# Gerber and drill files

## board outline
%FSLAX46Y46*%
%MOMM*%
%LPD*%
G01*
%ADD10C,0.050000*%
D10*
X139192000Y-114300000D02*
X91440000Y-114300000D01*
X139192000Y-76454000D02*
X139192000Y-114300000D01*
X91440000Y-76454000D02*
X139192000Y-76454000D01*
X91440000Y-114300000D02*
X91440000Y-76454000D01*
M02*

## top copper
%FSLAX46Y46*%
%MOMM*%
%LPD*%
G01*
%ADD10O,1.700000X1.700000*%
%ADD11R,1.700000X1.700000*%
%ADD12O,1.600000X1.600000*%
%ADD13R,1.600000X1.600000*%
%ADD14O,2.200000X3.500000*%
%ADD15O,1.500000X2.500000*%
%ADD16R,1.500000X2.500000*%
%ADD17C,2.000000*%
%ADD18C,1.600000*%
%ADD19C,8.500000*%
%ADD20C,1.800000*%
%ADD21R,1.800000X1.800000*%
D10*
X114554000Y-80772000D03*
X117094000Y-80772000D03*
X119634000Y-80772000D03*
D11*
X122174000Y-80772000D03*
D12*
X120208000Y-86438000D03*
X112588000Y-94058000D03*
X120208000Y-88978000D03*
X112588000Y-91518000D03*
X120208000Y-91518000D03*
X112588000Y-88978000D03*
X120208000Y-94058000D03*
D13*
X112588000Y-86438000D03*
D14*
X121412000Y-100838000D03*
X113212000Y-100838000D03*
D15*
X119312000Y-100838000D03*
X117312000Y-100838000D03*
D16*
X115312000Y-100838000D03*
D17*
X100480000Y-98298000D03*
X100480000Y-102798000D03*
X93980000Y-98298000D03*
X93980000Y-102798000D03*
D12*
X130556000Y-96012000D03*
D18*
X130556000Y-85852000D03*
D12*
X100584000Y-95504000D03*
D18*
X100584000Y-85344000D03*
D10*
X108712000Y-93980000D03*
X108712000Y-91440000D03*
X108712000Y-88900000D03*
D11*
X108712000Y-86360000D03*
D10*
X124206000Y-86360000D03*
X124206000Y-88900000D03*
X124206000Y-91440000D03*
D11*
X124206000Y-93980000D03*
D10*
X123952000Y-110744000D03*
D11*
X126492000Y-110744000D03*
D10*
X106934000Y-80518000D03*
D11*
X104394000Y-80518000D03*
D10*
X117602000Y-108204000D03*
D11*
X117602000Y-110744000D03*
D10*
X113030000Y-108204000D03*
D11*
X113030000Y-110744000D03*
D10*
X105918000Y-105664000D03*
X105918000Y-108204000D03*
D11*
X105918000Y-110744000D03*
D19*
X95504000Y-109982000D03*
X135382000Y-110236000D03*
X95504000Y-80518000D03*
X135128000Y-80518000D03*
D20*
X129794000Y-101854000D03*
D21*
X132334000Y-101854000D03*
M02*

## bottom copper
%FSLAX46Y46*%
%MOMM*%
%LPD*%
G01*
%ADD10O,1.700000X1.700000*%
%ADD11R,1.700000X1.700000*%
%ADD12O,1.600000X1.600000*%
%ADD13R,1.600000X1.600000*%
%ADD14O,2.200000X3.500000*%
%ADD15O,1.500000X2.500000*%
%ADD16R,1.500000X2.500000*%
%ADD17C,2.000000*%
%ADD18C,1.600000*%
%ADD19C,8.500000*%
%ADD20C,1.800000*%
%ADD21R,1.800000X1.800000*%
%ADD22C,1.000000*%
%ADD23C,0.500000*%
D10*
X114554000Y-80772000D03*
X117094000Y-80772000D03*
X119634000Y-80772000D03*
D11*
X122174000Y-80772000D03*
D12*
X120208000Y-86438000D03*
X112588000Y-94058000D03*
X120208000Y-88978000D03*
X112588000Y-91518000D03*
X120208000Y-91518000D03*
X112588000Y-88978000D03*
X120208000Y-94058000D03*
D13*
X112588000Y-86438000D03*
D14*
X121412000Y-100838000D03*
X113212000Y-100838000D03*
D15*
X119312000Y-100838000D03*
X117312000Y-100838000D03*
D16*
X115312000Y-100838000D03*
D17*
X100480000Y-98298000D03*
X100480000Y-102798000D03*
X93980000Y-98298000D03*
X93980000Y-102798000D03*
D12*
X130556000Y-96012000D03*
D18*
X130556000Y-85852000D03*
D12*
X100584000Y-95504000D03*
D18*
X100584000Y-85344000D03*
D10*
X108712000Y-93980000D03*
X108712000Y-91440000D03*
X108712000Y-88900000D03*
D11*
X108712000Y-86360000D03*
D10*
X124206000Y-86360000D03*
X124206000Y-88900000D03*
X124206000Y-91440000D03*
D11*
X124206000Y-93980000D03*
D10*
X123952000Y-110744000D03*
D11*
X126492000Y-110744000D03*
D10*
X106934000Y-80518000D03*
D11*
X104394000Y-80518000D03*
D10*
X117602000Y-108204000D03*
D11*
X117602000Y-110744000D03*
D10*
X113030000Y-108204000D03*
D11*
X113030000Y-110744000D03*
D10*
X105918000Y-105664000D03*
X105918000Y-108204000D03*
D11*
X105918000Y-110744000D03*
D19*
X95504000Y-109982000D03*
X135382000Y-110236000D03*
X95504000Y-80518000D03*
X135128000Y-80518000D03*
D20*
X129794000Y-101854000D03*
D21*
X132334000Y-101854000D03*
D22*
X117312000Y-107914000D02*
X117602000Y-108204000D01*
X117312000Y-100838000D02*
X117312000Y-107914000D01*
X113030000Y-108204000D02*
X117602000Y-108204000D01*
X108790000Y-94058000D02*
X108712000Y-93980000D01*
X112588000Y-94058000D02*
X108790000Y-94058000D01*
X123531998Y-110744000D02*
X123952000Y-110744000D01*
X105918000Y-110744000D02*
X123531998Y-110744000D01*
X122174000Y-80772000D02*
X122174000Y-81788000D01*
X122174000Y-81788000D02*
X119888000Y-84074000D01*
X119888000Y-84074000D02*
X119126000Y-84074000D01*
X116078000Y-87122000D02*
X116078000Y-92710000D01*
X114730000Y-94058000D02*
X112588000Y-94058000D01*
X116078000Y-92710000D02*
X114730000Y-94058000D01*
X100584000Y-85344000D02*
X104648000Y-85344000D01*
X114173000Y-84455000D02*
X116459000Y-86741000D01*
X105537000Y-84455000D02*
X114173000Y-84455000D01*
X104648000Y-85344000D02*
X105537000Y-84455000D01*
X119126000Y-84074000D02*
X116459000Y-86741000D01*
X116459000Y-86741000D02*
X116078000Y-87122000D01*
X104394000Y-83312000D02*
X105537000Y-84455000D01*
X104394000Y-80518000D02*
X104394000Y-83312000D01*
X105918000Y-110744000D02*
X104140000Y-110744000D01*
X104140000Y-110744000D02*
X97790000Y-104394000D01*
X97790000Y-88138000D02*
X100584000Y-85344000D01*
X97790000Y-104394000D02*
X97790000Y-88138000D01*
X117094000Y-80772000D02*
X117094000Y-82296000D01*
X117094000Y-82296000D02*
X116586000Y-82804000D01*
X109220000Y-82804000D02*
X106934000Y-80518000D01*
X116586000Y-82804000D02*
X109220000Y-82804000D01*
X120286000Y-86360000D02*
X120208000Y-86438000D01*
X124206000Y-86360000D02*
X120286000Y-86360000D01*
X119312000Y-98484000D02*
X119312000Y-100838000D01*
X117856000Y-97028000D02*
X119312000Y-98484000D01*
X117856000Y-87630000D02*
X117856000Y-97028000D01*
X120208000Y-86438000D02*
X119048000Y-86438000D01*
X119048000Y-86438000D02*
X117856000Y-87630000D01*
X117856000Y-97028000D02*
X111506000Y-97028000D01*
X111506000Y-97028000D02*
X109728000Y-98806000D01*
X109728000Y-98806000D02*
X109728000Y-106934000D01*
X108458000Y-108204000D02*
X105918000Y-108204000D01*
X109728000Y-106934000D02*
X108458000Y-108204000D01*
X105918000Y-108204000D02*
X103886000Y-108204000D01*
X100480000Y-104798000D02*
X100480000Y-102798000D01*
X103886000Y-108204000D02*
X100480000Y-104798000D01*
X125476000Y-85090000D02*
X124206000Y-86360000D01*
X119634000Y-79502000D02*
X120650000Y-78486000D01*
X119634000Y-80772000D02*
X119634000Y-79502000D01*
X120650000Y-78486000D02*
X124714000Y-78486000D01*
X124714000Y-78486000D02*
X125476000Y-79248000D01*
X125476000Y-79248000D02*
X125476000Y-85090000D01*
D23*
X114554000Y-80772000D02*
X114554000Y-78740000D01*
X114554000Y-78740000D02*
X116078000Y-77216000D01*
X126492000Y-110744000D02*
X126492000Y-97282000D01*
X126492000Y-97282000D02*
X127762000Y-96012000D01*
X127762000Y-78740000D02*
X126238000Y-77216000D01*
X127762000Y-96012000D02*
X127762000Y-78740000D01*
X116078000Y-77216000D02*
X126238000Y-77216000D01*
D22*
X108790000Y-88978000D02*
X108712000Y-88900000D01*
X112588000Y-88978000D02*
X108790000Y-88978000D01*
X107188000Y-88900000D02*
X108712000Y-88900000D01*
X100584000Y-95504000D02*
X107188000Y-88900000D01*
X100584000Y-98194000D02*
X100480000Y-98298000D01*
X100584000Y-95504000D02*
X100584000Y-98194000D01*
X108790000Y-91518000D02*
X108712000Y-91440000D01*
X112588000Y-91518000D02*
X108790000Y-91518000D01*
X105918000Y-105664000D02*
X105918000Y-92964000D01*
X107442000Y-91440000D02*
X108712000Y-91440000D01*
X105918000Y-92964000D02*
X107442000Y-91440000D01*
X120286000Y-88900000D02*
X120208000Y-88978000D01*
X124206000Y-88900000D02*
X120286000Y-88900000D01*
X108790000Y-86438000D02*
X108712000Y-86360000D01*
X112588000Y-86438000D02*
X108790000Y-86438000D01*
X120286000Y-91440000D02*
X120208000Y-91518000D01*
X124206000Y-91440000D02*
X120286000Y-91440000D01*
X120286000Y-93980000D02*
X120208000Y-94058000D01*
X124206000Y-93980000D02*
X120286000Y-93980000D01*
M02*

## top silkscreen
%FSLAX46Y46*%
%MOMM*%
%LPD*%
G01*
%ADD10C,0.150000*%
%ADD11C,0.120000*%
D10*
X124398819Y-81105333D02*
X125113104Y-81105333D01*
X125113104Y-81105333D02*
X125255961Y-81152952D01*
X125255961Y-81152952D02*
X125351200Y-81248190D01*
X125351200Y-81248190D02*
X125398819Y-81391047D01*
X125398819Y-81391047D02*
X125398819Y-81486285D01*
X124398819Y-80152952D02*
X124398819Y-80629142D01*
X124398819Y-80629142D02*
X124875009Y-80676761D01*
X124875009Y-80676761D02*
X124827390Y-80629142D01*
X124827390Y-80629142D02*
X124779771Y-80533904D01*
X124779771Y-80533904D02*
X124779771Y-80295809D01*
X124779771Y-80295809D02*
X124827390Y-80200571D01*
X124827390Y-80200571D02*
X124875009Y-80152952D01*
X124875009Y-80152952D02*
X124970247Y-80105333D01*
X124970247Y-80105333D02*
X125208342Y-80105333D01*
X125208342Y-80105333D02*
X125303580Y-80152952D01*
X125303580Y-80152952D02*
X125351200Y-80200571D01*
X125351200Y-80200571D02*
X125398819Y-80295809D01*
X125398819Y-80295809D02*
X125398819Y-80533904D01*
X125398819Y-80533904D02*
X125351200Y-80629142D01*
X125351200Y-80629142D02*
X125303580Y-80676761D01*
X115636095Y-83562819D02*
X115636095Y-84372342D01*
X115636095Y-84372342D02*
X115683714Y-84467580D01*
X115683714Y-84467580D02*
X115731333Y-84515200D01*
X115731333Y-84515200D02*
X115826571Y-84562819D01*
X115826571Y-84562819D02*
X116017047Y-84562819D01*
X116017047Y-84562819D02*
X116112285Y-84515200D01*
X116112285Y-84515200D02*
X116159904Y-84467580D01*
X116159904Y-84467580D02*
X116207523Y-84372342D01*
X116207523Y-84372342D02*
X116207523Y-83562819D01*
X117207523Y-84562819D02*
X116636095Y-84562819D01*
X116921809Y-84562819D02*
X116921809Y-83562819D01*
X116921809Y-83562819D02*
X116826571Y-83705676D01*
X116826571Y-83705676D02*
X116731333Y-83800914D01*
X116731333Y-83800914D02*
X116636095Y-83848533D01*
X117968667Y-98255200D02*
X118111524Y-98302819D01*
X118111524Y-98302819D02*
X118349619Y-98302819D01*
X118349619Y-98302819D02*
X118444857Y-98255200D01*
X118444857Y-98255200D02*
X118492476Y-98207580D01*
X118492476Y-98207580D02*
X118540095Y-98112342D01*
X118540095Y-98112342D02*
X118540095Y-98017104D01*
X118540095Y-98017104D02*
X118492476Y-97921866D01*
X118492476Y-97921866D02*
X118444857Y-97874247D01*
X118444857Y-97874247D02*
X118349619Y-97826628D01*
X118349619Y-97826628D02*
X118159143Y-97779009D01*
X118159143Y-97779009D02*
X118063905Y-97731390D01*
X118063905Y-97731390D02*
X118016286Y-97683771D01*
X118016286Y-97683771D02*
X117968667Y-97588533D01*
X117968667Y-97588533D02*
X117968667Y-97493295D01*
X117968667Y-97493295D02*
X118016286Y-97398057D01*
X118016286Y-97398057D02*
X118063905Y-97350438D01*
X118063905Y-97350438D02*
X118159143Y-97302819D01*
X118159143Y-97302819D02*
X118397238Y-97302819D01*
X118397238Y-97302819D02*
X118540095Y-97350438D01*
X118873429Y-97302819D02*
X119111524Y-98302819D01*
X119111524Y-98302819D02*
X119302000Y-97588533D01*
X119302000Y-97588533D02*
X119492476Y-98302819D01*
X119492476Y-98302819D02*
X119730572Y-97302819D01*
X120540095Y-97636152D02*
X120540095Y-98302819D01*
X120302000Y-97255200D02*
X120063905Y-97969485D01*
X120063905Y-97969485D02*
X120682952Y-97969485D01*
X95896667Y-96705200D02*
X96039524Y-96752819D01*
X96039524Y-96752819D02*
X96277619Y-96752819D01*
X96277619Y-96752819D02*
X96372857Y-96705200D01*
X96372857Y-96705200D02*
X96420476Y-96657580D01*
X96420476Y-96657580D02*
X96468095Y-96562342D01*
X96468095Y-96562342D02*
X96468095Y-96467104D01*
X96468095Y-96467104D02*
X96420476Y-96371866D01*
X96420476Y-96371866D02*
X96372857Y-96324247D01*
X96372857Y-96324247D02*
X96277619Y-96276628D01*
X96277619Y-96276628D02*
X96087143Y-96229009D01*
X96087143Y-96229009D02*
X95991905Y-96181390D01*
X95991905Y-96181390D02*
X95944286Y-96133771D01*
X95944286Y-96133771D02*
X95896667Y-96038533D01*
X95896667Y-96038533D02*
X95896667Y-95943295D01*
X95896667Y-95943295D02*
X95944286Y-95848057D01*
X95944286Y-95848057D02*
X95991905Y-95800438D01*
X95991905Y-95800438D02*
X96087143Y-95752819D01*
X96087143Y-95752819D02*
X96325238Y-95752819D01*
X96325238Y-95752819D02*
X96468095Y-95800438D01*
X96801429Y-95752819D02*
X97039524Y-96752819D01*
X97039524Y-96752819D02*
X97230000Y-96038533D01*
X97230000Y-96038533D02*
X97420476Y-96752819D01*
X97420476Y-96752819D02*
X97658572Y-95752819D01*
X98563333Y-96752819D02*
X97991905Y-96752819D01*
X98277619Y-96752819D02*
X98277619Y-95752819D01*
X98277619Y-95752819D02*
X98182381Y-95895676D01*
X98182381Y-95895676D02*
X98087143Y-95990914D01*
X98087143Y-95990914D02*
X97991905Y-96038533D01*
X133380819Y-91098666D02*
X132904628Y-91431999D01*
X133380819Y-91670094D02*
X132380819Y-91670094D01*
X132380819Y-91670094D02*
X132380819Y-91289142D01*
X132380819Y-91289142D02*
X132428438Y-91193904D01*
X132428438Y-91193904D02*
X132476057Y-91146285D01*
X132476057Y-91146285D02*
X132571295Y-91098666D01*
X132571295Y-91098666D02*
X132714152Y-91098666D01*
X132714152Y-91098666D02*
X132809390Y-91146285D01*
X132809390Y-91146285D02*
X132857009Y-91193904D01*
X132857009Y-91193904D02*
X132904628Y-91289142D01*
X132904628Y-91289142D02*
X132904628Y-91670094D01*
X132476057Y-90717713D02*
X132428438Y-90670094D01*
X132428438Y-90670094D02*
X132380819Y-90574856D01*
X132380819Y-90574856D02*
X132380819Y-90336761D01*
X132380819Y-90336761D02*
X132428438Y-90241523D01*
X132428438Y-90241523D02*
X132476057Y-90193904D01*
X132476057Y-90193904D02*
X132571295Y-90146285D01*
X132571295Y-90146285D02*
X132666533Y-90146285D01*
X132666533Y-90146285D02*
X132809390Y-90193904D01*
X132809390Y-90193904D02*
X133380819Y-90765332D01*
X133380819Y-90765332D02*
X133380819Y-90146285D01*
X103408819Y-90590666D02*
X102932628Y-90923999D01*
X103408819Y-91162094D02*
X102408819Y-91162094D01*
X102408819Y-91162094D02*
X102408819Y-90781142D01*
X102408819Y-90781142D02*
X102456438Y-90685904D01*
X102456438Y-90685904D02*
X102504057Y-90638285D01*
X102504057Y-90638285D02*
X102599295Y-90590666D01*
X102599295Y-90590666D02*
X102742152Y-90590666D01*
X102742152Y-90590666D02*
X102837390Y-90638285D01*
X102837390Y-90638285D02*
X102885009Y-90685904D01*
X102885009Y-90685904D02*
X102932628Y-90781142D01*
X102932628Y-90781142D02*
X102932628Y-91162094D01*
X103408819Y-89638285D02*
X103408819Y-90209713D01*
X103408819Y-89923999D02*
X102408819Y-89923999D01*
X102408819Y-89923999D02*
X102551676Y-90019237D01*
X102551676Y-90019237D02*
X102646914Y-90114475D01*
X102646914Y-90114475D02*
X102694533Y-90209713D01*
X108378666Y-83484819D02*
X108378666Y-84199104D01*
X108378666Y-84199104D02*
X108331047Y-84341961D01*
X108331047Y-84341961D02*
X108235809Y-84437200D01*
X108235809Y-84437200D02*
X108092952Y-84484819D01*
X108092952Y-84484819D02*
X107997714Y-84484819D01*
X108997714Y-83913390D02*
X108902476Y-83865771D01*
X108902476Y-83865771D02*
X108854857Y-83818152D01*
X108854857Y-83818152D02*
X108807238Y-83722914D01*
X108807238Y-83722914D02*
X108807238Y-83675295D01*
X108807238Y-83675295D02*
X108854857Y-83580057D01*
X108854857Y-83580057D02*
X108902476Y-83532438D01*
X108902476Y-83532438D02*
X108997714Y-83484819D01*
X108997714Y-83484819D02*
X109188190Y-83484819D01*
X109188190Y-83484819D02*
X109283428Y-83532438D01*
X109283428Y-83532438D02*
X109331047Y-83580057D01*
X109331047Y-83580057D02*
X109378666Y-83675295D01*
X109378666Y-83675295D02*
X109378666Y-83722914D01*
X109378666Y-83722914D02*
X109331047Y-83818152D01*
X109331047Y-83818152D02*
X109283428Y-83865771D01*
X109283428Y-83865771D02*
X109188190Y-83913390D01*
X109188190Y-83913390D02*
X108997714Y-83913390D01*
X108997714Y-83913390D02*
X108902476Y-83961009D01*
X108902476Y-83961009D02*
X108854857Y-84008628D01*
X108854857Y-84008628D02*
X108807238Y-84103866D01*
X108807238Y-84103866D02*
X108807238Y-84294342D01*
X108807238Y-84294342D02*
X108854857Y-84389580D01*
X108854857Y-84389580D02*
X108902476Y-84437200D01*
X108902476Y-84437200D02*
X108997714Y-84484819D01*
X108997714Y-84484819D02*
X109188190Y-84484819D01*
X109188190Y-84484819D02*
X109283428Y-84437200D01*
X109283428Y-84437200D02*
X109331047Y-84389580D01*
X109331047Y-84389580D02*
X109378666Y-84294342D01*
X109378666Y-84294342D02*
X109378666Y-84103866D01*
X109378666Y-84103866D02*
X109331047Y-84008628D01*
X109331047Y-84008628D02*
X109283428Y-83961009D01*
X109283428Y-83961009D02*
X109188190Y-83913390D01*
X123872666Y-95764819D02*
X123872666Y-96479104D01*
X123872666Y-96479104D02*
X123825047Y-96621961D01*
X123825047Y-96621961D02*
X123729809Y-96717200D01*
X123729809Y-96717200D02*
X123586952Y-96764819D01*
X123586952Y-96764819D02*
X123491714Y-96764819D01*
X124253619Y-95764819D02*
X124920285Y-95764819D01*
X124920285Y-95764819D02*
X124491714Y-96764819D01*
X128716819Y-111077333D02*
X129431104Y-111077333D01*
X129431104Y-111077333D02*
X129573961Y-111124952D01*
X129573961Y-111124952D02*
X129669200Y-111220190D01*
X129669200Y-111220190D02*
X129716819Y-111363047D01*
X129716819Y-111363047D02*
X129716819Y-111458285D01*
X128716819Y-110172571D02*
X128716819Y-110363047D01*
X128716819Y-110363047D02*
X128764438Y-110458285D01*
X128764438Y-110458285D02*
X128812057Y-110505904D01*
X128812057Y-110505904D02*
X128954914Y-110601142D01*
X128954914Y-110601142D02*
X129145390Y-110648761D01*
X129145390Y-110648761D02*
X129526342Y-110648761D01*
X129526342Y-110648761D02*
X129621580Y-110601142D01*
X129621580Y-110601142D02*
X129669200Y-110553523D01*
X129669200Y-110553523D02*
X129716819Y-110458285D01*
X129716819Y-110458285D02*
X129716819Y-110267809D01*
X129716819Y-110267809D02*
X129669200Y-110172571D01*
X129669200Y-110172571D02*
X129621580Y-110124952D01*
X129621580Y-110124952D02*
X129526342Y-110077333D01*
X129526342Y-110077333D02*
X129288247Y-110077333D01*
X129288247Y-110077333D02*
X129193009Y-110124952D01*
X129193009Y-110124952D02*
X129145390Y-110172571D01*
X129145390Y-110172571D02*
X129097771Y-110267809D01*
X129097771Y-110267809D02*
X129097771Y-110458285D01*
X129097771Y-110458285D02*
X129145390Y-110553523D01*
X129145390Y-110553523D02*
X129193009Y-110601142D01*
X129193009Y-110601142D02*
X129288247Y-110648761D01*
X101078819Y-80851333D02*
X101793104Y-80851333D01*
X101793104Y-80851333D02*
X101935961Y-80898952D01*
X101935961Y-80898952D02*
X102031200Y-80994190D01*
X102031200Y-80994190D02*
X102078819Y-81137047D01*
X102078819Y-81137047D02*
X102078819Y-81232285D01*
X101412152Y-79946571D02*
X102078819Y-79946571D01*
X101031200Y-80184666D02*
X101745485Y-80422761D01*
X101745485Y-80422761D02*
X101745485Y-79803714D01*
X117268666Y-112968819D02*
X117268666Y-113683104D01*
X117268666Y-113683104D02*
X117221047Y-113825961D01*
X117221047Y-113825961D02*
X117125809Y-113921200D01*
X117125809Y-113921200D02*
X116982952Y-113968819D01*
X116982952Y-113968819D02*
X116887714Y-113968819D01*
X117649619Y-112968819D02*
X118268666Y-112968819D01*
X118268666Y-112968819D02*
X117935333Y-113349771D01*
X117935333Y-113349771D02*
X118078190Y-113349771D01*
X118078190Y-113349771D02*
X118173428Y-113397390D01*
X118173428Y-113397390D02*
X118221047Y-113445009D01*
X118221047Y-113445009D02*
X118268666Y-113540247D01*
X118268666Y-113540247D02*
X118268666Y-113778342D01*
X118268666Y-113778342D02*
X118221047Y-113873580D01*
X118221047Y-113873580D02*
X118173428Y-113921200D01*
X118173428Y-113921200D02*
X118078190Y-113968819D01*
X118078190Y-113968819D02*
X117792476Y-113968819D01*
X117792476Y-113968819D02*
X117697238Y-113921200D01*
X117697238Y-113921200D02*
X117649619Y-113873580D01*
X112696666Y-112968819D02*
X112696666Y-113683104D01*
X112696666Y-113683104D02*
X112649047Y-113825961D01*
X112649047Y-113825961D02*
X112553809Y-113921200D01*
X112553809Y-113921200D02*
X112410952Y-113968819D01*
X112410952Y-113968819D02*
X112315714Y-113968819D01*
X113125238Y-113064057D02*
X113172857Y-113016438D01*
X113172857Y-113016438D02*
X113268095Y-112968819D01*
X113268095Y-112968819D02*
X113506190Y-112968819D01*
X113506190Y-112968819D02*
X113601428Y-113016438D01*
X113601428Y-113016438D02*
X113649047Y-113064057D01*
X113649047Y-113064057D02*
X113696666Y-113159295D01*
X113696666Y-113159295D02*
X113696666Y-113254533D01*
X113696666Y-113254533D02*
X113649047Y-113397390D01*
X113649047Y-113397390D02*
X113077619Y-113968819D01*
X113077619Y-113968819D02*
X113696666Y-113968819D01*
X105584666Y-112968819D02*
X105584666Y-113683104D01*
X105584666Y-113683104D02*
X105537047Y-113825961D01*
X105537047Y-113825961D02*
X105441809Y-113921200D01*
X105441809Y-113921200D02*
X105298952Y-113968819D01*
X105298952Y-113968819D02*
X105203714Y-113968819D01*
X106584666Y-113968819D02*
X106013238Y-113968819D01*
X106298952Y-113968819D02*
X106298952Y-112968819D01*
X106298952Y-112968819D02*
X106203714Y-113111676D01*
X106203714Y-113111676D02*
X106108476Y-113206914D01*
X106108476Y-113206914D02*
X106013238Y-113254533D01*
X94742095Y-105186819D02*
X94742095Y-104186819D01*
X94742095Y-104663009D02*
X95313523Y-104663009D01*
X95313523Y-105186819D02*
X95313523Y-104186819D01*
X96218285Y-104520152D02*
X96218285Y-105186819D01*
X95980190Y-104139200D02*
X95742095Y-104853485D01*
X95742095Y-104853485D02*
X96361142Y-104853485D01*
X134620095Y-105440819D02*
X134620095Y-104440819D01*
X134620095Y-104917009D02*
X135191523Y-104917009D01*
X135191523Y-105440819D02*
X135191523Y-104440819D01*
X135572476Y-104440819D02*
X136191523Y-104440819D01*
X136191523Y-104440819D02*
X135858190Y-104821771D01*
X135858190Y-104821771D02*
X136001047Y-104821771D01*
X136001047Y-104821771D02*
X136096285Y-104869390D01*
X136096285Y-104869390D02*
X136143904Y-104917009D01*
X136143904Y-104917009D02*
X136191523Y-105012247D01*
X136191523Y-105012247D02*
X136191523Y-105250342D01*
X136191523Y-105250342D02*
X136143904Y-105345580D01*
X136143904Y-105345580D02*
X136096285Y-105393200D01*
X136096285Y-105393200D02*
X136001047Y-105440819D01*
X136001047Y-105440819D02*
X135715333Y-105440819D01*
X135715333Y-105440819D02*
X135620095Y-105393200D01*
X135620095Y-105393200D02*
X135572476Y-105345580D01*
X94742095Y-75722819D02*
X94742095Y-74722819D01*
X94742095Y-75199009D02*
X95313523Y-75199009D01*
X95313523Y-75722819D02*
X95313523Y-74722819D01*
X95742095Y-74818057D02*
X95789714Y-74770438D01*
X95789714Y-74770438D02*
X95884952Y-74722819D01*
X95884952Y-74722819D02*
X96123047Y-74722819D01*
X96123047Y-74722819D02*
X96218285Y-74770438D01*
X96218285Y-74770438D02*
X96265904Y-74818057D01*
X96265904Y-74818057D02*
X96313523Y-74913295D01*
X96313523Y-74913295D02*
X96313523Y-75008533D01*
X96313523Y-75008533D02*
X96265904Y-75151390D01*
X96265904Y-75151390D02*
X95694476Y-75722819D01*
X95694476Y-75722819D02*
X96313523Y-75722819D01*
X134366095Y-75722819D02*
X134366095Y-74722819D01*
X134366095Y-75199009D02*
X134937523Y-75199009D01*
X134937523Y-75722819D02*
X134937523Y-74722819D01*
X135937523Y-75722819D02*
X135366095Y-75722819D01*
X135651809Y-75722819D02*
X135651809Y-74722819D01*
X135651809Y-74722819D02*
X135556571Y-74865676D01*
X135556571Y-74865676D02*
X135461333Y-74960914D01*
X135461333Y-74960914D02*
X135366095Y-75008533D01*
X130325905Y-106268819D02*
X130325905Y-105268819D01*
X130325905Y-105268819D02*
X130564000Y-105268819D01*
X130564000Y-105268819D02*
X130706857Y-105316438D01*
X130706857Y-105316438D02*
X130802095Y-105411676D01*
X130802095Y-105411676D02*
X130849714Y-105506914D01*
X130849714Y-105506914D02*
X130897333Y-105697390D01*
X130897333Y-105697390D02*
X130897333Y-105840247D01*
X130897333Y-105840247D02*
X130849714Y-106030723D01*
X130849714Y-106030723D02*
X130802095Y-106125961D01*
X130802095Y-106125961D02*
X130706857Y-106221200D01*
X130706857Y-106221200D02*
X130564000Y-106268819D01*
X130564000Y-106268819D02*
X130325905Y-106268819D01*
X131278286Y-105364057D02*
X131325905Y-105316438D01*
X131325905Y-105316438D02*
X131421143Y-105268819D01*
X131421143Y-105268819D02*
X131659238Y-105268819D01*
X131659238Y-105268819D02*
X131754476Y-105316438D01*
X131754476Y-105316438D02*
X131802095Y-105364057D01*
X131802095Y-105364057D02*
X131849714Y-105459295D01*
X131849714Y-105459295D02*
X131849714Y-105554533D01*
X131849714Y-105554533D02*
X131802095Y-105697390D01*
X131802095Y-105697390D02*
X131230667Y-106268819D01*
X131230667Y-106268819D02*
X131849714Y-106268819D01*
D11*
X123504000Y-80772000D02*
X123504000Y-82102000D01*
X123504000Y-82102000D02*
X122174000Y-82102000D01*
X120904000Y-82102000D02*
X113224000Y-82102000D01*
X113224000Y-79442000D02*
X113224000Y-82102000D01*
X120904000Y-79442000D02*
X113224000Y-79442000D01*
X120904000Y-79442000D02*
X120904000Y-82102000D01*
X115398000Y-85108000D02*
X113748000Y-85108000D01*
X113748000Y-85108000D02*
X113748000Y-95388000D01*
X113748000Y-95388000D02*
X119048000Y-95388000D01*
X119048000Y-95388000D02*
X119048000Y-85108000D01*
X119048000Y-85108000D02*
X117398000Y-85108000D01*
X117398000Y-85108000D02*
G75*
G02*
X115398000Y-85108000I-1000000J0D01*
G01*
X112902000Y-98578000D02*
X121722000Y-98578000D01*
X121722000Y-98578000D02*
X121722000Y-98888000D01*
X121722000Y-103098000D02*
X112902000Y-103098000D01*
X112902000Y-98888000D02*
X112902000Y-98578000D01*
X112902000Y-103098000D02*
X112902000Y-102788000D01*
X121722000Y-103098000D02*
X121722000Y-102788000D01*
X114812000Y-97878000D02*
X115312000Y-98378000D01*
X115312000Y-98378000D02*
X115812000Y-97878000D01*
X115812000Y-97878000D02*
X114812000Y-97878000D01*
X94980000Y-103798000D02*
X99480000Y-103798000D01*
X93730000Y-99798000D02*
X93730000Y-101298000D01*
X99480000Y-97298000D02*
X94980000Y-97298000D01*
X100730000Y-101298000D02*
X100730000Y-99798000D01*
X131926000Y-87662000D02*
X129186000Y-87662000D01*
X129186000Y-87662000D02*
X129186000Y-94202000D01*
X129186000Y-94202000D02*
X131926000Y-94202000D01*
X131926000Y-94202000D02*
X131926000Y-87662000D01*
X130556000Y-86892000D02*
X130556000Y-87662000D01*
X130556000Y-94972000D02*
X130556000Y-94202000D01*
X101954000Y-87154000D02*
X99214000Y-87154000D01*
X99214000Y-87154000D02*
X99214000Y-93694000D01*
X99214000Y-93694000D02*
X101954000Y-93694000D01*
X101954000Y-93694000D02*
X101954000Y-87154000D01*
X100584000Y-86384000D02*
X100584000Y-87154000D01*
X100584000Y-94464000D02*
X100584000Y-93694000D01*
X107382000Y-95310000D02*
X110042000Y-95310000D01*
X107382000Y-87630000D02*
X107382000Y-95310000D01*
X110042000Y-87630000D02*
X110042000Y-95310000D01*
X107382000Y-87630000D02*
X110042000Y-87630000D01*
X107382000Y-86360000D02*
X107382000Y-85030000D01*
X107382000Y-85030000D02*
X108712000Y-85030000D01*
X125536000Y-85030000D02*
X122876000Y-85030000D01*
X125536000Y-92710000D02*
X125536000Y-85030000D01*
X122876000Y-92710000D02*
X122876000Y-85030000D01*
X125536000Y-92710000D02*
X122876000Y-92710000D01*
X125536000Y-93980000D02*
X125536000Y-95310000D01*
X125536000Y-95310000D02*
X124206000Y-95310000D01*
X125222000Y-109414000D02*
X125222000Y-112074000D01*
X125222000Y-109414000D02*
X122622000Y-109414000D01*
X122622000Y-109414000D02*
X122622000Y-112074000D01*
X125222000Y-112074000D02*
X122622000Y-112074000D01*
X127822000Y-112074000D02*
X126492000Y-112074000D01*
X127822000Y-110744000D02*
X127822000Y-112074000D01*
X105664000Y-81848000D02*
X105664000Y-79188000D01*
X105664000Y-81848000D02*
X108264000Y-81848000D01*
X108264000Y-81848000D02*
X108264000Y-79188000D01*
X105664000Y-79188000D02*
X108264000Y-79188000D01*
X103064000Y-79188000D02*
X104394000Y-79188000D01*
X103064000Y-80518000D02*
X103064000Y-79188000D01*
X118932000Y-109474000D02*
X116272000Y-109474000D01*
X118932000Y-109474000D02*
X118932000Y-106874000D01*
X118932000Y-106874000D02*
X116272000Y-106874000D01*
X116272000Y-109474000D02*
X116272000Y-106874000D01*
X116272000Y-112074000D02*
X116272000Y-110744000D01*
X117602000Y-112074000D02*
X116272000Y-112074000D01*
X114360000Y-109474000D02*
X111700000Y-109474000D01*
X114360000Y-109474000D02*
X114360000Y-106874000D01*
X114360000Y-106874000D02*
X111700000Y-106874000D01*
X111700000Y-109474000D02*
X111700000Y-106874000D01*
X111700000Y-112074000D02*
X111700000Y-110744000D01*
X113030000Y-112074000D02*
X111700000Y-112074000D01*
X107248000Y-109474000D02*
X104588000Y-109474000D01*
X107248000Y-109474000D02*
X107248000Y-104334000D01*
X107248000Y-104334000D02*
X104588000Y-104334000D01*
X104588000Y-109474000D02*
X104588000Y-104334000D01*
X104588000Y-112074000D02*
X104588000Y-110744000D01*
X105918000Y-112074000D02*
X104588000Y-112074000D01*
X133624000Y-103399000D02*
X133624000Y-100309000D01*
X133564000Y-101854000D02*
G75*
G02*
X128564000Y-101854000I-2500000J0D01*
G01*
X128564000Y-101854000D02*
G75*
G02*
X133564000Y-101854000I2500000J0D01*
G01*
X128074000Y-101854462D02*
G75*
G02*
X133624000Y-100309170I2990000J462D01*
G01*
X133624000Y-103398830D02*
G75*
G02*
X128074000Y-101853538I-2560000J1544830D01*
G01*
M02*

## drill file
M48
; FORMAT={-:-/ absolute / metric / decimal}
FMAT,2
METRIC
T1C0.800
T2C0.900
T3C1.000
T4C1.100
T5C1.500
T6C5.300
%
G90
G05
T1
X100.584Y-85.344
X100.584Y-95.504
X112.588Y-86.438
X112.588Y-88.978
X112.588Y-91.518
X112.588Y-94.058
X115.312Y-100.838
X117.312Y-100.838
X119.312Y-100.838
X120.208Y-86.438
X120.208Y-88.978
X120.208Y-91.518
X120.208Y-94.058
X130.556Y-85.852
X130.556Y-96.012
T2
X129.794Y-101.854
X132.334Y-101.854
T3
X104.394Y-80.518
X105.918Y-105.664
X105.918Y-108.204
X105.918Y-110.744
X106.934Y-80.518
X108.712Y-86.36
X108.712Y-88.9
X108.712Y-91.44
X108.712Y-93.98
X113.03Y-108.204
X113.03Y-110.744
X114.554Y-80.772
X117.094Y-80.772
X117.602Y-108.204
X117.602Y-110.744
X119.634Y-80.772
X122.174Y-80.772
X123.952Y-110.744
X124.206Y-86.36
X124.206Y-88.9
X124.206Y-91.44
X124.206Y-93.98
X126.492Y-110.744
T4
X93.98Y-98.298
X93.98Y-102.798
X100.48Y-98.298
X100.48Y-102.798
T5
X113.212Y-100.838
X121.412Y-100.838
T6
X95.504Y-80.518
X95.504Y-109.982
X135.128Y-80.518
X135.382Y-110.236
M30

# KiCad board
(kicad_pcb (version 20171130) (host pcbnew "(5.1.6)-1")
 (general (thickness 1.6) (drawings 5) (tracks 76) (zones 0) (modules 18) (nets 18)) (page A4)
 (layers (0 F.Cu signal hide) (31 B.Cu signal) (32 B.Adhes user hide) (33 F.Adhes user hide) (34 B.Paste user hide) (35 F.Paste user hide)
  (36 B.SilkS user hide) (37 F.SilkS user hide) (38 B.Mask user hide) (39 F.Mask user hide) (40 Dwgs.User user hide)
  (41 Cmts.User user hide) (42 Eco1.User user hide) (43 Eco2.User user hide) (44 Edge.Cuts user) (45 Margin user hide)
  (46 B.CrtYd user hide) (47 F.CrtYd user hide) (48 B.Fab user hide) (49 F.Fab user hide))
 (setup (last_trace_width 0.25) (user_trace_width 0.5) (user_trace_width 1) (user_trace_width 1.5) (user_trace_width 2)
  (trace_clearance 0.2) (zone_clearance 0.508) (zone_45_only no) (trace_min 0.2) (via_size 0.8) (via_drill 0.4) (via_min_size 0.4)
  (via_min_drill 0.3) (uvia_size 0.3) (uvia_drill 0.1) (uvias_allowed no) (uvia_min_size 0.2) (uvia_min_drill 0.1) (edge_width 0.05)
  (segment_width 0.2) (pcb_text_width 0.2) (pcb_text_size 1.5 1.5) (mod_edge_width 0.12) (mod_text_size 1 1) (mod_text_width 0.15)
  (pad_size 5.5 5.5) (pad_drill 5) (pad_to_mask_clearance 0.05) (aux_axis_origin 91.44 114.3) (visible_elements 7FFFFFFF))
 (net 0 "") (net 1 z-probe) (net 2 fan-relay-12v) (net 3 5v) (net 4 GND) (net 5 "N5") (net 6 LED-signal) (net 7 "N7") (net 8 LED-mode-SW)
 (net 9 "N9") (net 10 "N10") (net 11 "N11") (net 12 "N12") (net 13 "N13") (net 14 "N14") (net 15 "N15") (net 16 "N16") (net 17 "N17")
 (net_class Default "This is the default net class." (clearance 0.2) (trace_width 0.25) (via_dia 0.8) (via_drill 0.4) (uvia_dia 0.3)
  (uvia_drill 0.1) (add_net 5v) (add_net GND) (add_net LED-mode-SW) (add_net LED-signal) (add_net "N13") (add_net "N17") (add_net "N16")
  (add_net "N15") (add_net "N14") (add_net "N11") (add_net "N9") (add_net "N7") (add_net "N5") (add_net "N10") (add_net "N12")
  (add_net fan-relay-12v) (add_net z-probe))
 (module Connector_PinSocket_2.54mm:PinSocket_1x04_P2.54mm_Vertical (layer F.Cu) (at 122.174 80.772 270)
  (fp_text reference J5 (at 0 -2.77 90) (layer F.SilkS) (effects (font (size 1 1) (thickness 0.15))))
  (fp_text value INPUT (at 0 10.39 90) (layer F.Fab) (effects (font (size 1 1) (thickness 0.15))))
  (fp_line (start 0 -1.33) (end 1.33 -1.33) (layer F.SilkS) (width 0.12))
  (fp_line (start 1.33 -1.33) (end 1.33 0) (layer F.SilkS) (width 0.12))
  (fp_line (start 1.33 1.27) (end 1.33 8.95) (layer F.SilkS) (width 0.12))
  (fp_line (start -1.33 8.95) (end 1.33 8.95) (layer F.SilkS) (width 0.12))
  (fp_line (start -1.33 1.27) (end -1.33 8.95) (layer F.SilkS) (width 0.12))
  (fp_line (start -1.33 1.27) (end 1.33 1.27) (layer F.SilkS) (width 0.12))
  (pad 4 thru_hole oval (at 0 7.62 270) (size 1.7 1.7) (drill 1) (layers *.Cu *.Mask) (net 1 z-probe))
  (pad 3 thru_hole oval (at 0 5.08 270) (size 1.7 1.7) (drill 1) (layers *.Cu *.Mask) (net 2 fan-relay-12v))
  (pad 2 thru_hole oval (at 0 2.54 270) (size 1.7 1.7) (drill 1) (layers *.Cu *.Mask) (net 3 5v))
  (pad 1 thru_hole rect (at 0 0 270) (size 1.7 1.7) (drill 1) (layers *.Cu *.Mask) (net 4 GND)))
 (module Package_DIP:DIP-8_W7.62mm (layer F.Cu) (at 112.588 86.438)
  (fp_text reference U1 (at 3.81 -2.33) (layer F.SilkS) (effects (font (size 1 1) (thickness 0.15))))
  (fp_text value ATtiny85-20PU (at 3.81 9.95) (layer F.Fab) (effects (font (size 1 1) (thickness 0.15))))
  (fp_line (start 2.81 -1.33) (end 1.16 -1.33) (layer F.SilkS) (width 0.12))
  (fp_line (start 1.16 -1.33) (end 1.16 8.95) (layer F.SilkS) (width 0.12))
  (fp_line (start 1.16 8.95) (end 6.46 8.95) (layer F.SilkS) (width 0.12))
  (fp_line (start 6.46 8.95) (end 6.46 -1.33) (layer F.SilkS) (width 0.12))
  (fp_line (start 6.46 -1.33) (end 4.81 -1.33) (layer F.SilkS) (width 0.12))
  (fp_arc (start 3.81 -1.33) (end 2.81 -1.33) (angle -180) (layer F.SilkS) (width 0.12))
  (pad 8 thru_hole oval (at 7.62 0) (size 1.6 1.6) (drill 0.8) (layers *.Cu *.Mask) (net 3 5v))
  (pad 4 thru_hole oval (at 0 7.62) (size 1.6 1.6) (drill 0.8) (layers *.Cu *.Mask) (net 4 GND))
  (pad 7 thru_hole oval (at 7.62 2.54) (size 1.6 1.6) (drill 0.8) (layers *.Cu *.Mask) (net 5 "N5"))
  (pad 3 thru_hole oval (at 0 5.08) (size 1.6 1.6) (drill 0.8) (layers *.Cu *.Mask) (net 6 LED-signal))
  (pad 6 thru_hole oval (at 7.62 5.08) (size 1.6 1.6) (drill 0.8) (layers *.Cu *.Mask) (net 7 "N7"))
  (pad 2 thru_hole oval (at 0 2.54) (size 1.6 1.6) (drill 0.8) (layers *.Cu *.Mask) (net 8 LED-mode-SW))
  (pad 5 thru_hole oval (at 7.62 7.62) (size 1.6 1.6) (drill 0.8) (layers *.Cu *.Mask) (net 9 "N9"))
  (pad 1 thru_hole rect (at 0 0) (size 1.6 1.6) (drill 0.8) (layers *.Cu *.Mask) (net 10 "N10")))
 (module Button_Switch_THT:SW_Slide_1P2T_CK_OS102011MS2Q (layer F.Cu) (at 115.312 100.838)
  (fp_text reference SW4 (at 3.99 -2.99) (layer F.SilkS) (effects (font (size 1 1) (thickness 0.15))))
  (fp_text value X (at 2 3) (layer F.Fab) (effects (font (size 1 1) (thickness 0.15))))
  (fp_line (start -2.41 -2.26) (end 6.41 -2.26) (layer F.SilkS) (width 0.12))
  (fp_line (start 6.41 -2.26) (end 6.41 -1.95) (layer F.SilkS) (width 0.12))
  (fp_line (start 6.41 2.26) (end -2.41 2.26) (layer F.SilkS) (width 0.12))
  (fp_line (start -2.41 -1.95) (end -2.41 -2.26) (layer F.SilkS) (width 0.12))
  (fp_line (start -2.41 2.26) (end -2.41 1.95) (layer F.SilkS) (width 0.12))
  (fp_line (start 6.41 2.26) (end 6.41 1.95) (layer F.SilkS) (width 0.12))
  (fp_line (start -0.5 -2.96) (end 0 -2.46) (layer F.SilkS) (width 0.12))
  (fp_line (start 0 -2.46) (end 0.5 -2.96) (layer F.SilkS) (width 0.12))
  (fp_line (start 0.5 -2.96) (end -0.5 -2.96) (layer F.SilkS) (width 0.12))
  (pad "" thru_hole oval (at 6.1 0) (size 2.2 3.5) (drill 1.5) (layers *.Cu *.Mask))
  (pad "" thru_hole oval (at -2.1 0) (size 2.2 3.5) (drill 1.5) (layers *.Cu *.Mask))
  (pad 3 thru_hole oval (at 4 0) (size 1.5 2.5) (drill 0.8) (layers *.Cu *.Mask) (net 3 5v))
  (pad 2 thru_hole oval (at 2 0) (size 1.5 2.5) (drill 0.8) (layers *.Cu *.Mask) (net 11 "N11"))
  (pad 1 thru_hole rect (at 0 0) (size 1.5 2.5) (drill 0.8) (layers *.Cu *.Mask) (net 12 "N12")))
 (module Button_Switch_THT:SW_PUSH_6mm (layer F.Cu) (at 93.98 98.298)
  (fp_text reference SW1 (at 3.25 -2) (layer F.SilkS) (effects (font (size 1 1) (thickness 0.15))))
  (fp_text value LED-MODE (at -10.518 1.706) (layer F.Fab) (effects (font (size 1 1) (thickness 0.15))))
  (fp_line (start 1 5.5) (end 5.5 5.5) (layer F.SilkS) (width 0.12))
  (fp_line (start -0.25 1.5) (end -0.25 3) (layer F.SilkS) (width 0.12))
  (fp_line (start 5.5 -1) (end 1 -1) (layer F.SilkS) (width 0.12))
  (fp_line (start 6.75 3) (end 6.75 1.5) (layer F.SilkS) (width 0.12))
  (pad 1 thru_hole circle (at 6.5 0 90) (size 2 2) (drill 1.1) (layers *.Cu *.Mask) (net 8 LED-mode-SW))
  (pad 2 thru_hole circle (at 6.5 4.5 90) (size 2 2) (drill 1.1) (layers *.Cu *.Mask) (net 3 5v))
  (pad 1 thru_hole circle (at 0 0 90) (size 2 2) (drill 1.1) (layers *.Cu *.Mask) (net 8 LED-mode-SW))
  (pad 2 thru_hole circle (at 0 4.5 90) (size 2 2) (drill 1.1) (layers *.Cu *.Mask) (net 3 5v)))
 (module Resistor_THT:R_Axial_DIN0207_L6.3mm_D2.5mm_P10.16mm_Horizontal (layer F.Cu) (at 130.556 85.852 270)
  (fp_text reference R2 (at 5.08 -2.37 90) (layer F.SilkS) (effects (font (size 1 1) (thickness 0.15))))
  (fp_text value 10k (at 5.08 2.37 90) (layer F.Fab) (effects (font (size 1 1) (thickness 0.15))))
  (fp_line (start 1.81 -1.37) (end 1.81 1.37) (layer F.SilkS) (width 0.12))
  (fp_line (start 1.81 1.37) (end 8.35 1.37) (layer F.SilkS) (width 0.12))
  (fp_line (start 8.35 1.37) (end 8.35 -1.37) (layer F.SilkS) (width 0.12))
  (fp_line (start 8.35 -1.37) (end 1.81 -1.37) (layer F.SilkS) (width 0.12))
  (fp_line (start 1.04 0) (end 1.81 0) (layer F.SilkS) (width 0.12))
  (fp_line (start 9.12 0) (end 8.35 0) (layer F.SilkS) (width 0.12))
  (pad 2 thru_hole oval (at 10.16 0 270) (size 1.6 1.6) (drill 0.8) (layers *.Cu *.Mask) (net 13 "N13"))
  (pad 1 thru_hole circle (at 0 0 270) (size 1.6 1.6) (drill 0.8) (layers *.Cu *.Mask) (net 3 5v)))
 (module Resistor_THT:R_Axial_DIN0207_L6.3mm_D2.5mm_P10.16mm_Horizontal (layer F.Cu) (at 100.584 85.344 270)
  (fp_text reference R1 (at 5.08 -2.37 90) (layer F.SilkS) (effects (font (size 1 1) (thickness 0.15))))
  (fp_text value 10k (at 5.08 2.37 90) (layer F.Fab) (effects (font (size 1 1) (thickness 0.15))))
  (fp_line (start 1.81 -1.37) (end 1.81 1.37) (layer F.SilkS) (width 0.12))
  (fp_line (start 1.81 1.37) (end 8.35 1.37) (layer F.SilkS) (width 0.12))
  (fp_line (start 8.35 1.37) (end 8.35 -1.37) (layer F.SilkS) (width 0.12))
  (fp_line (start 8.35 -1.37) (end 1.81 -1.37) (layer F.SilkS) (width 0.12))
  (fp_line (start 1.04 0) (end 1.81 0) (layer F.SilkS) (width 0.12))
  (fp_line (start 9.12 0) (end 8.35 0) (layer F.SilkS) (width 0.12))
  (pad 2 thru_hole oval (at 10.16 0 270) (size 1.6 1.6) (drill 0.8) (layers *.Cu *.Mask) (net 8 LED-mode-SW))
  (pad 1 thru_hole circle (at 0 0 270) (size 1.6 1.6) (drill 0.8) (layers *.Cu *.Mask) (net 4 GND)))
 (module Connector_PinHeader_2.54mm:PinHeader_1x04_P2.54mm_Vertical (layer F.Cu) (at 108.712 86.36)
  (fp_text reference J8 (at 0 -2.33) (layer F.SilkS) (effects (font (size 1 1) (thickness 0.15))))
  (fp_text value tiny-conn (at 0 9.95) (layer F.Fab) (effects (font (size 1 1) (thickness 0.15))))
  (fp_line (start -1.33 8.95) (end 1.33 8.95) (layer F.SilkS) (width 0.12))
  (fp_line (start -1.33 1.27) (end -1.33 8.95) (layer F.SilkS) (width 0.12))
  (fp_line (start 1.33 1.27) (end 1.33 8.95) (layer F.SilkS) (width 0.12))
  (fp_line (start -1.33 1.27) (end 1.33 1.27) (layer F.SilkS) (width 0.12))
  (fp_line (start -1.33 0) (end -1.33 -1.33) (layer F.SilkS) (width 0.12))
  (fp_line (start -1.33 -1.33) (end 0 -1.33) (layer F.SilkS) (width 0.12))
  (pad 4 thru_hole oval (at 0 7.62) (size 1.7 1.7) (drill 1) (layers *.Cu *.Mask) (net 4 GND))
  (pad 3 thru_hole oval (at 0 5.08) (size 1.7 1.7) (drill 1) (layers *.Cu *.Mask) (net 6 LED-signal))
  (pad 2 thru_hole oval (at 0 2.54) (size 1.7 1.7) (drill 1) (layers *.Cu *.Mask) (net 8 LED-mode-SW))
  (pad 1 thru_hole rect (at 0 0) (size 1.7 1.7) (drill 1) (layers *.Cu *.Mask) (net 10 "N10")))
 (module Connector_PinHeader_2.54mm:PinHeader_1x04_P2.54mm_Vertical (layer F.Cu) (at 124.206 93.98 180)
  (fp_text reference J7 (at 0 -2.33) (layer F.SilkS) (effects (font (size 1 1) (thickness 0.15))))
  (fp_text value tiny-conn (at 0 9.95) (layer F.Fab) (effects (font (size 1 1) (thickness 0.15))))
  (fp_line (start -1.33 8.95) (end 1.33 8.95) (layer F.SilkS) (width 0.12))
  (fp_line (start -1.33 1.27) (end -1.33 8.95) (layer F.SilkS) (width 0.12))
  (fp_line (start 1.33 1.27) (end 1.33 8.95) (layer F.SilkS) (width 0.12))
  (fp_line (start -1.33 1.27) (end 1.33 1.27) (layer F.SilkS) (width 0.12))
  (fp_line (start -1.33 0) (end -1.33 -1.33) (layer F.SilkS) (width 0.12))
  (fp_line (start -1.33 -1.33) (end 0 -1.33) (layer F.SilkS) (width 0.12))
  (pad 4 thru_hole oval (at 0 7.62 180) (size 1.7 1.7) (drill 1) (layers *.Cu *.Mask) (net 3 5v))
  (pad 3 thru_hole oval (at 0 5.08 180) (size 1.7 1.7) (drill 1) (layers *.Cu *.Mask) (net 5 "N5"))
  (pad 2 thru_hole oval (at 0 2.54 180) (size 1.7 1.7) (drill 1) (layers *.Cu *.Mask) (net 7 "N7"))
  (pad 1 thru_hole rect (at 0 0 180) (size 1.7 1.7) (drill 1) (layers *.Cu *.Mask) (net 9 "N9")))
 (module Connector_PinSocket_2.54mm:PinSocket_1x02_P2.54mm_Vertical (layer F.Cu) (at 126.492 110.744 270)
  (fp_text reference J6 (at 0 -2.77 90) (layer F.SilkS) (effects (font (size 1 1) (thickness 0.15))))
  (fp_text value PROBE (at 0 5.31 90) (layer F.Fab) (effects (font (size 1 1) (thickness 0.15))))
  (fp_line (start -1.33 1.27) (end 1.33 1.27) (layer F.SilkS) (width 0.12))
  (fp_line (start -1.33 1.27) (end -1.33 3.87) (layer F.SilkS) (width 0.12))
  (fp_line (start -1.33 3.87) (end 1.33 3.87) (layer F.SilkS) (width 0.12))
  (fp_line (start 1.33 1.27) (end 1.33 3.87) (layer F.SilkS) (width 0.12))
  (fp_line (start 1.33 -1.33) (end 1.33 0) (layer F.SilkS) (width 0.12))
  (fp_line (start 0 -1.33) (end 1.33 -1.33) (layer F.SilkS) (width 0.12))
  (pad 2 thru_hole oval (at 0 2.54 270) (size 1.7 1.7) (drill 1) (layers *.Cu *.Mask) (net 4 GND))
  (pad 1 thru_hole rect (at 0 0 270) (size 1.7 1.7) (drill 1) (layers *.Cu *.Mask) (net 1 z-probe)))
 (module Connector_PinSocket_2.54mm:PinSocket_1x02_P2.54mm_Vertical (layer F.Cu) (at 104.394 80.518 90)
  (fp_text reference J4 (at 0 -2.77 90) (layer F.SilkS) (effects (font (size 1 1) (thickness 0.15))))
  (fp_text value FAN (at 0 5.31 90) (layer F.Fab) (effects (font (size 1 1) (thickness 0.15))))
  (fp_line (start -1.33 1.27) (end 1.33 1.27) (layer F.SilkS) (width 0.12))
  (fp_line (start -1.33 1.27) (end -1.33 3.87) (layer F.SilkS) (width 0.12))
  (fp_line (start -1.33 3.87) (end 1.33 3.87) (layer F.SilkS) (width 0.12))
  (fp_line (start 1.33 1.27) (end 1.33 3.87) (layer F.SilkS) (width 0.12))
  (fp_line (start 1.33 -1.33) (end 1.33 0) (layer F.SilkS) (width 0.12))
  (fp_line (start 0 -1.33) (end 1.33 -1.33) (layer F.SilkS) (width 0.12))
  (pad 2 thru_hole oval (at 0 2.54 90) (size 1.7 1.7) (drill 1) (layers *.Cu *.Mask) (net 2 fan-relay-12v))
  (pad 1 thru_hole rect (at 0 0 90) (size 1.7 1.7) (drill 1) (layers *.Cu *.Mask) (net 4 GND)))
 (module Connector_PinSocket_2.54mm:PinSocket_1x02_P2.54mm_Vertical (layer F.Cu) (at 117.602 110.744 180)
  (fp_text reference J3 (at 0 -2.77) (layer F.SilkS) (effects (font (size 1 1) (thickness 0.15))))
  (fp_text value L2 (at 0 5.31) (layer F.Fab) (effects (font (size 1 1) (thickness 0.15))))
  (fp_line (start -1.33 1.27) (end 1.33 1.27) (layer F.SilkS) (width 0.12))
  (fp_line (start -1.33 1.27) (end -1.33 3.87) (layer F.SilkS) (width 0.12))
  (fp_line (start -1.33 3.87) (end 1.33 3.87) (layer F.SilkS) (width 0.12))
  (fp_line (start 1.33 1.27) (end 1.33 3.87) (layer F.SilkS) (width 0.12))
  (fp_line (start 1.33 -1.33) (end 1.33 0) (layer F.SilkS) (width 0.12))
  (fp_line (start 0 -1.33) (end 1.33 -1.33) (layer F.SilkS) (width 0.12))
  (pad 2 thru_hole oval (at 0 2.54 180) (size 1.7 1.7) (drill 1) (layers *.Cu *.Mask) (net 11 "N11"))
  (pad 1 thru_hole rect (at 0 0 180) (size 1.7 1.7) (drill 1) (layers *.Cu *.Mask) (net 4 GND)))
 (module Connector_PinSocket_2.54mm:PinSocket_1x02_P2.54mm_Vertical (layer F.Cu) (at 113.03 110.744 180)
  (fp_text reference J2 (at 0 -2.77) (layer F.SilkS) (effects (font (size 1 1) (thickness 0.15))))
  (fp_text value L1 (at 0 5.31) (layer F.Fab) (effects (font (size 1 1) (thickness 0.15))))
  (fp_line (start -1.33 1.27) (end 1.33 1.27) (layer F.SilkS) (width 0.12))
  (fp_line (start -1.33 1.27) (end -1.33 3.87) (layer F.SilkS) (width 0.12))
  (fp_line (start -1.33 3.87) (end 1.33 3.87) (layer F.SilkS) (width 0.12))
  (fp_line (start 1.33 1.27) (end 1.33 3.87) (layer F.SilkS) (width 0.12))
  (fp_line (start 1.33 -1.33) (end 1.33 0) (layer F.SilkS) (width 0.12))
  (fp_line (start 0 -1.33) (end 1.33 -1.33) (layer F.SilkS) (width 0.12))
  (pad 2 thru_hole oval (at 0 2.54 180) (size 1.7 1.7) (drill 1) (layers *.Cu *.Mask) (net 11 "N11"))
  (pad 1 thru_hole rect (at 0 0 180) (size 1.7 1.7) (drill 1) (layers *.Cu *.Mask) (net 4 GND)))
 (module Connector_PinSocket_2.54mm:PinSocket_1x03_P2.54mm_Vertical (layer F.Cu) (at 105.918 110.744 180)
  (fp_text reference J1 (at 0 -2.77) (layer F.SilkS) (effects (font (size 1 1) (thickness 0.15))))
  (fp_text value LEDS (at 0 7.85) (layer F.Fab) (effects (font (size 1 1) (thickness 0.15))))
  (fp_line (start -1.33 1.27) (end 1.33 1.27) (layer F.SilkS) (width 0.12))
  (fp_line (start -1.33 1.27) (end -1.33 6.41) (layer F.SilkS) (width 0.12))
  (fp_line (start -1.33 6.41) (end 1.33 6.41) (layer F.SilkS) (width 0.12))
  (fp_line (start 1.33 1.27) (end 1.33 6.41) (layer F.SilkS) (width 0.12))
  (fp_line (start 1.33 -1.33) (end 1.33 0) (layer F.SilkS) (width 0.12))
  (fp_line (start 0 -1.33) (end 1.33 -1.33) (layer F.SilkS) (width 0.12))
  (pad 3 thru_hole oval (at 0 5.08 180) (size 1.7 1.7) (drill 1) (layers *.Cu *.Mask) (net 6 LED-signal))
  (pad 2 thru_hole oval (at 0 2.54 180) (size 1.7 1.7) (drill 1) (layers *.Cu *.Mask) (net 3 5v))
  (pad 1 thru_hole rect (at 0 0 180) (size 1.7 1.7) (drill 1) (layers *.Cu *.Mask) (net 4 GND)))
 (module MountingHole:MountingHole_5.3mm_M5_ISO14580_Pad (layer F.Cu) (at 95.504 109.982)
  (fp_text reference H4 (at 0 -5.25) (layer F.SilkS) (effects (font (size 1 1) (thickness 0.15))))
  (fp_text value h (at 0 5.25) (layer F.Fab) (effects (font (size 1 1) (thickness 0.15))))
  (pad 1 thru_hole circle (at 0 0) (size 8.5 8.5) (drill 5.3) (layers *.Cu *.Mask) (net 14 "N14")))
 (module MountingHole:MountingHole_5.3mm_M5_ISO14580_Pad (layer F.Cu) (at 135.382 110.236)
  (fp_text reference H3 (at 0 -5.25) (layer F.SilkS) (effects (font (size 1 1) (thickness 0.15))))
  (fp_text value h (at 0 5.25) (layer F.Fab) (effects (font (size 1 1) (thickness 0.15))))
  (pad 1 thru_hole circle (at 0 0) (size 8.5 8.5) (drill 5.3) (layers *.Cu *.Mask) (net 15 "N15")))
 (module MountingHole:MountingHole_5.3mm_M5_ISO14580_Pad (layer F.Cu) (at 95.504 80.518)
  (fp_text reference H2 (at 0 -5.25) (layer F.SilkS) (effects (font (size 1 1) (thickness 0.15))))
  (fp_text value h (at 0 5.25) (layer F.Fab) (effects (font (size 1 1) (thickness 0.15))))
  (pad 1 thru_hole circle (at 0 0) (size 8.5 8.5) (drill 5.3) (layers *.Cu *.Mask) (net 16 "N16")))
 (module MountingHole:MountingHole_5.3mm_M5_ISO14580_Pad (layer F.Cu) (at 135.128 80.518)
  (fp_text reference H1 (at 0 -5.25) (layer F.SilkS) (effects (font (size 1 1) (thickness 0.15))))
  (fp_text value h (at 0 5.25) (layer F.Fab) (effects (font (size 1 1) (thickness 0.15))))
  (pad 1 thru_hole circle (at 0 0) (size 8.5 8.5) (drill 5.3) (layers *.Cu *.Mask) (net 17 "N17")))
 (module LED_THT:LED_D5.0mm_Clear (layer F.Cu) (at 132.334 101.854 180)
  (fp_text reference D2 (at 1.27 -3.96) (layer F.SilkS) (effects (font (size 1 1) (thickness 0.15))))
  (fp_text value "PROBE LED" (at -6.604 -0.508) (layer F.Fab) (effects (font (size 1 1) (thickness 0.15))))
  (fp_line (start -1.29 -1.545) (end -1.29 1.545) (layer F.SilkS) (width 0.12))
  (fp_circle (center 1.27 0) (end 3.77 0) (layer F.SilkS) (width 0.12))
  (fp_arc (start 1.27 0) (end -1.29 1.54483) (angle -148.9) (layer F.SilkS) (width 0.12))
  (fp_arc (start 1.27 0) (end -1.29 -1.54483) (angle 148.9) (layer F.SilkS) (width 0.12))
  (pad 2 thru_hole circle (at 2.54 0 180) (size 1.8 1.8) (drill 0.9) (layers *.Cu *.Mask) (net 1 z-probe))
  (pad 1 thru_hole rect (at 0 0 180) (size 1.8 1.8) (drill 0.9) (layers *.Cu *.Mask) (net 13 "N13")))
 (gr_line (start 139.192 114.3) (end 91.44 114.3) (layer Edge.Cuts) (width 0.05))
 (gr_line (start 139.192 76.454) (end 139.192 114.3) (layer Edge.Cuts) (width 0.05))
 (gr_line (start 91.44 76.454) (end 139.192 76.454) (layer Edge.Cuts) (width 0.05))
 (gr_line (start 91.44 114.3) (end 91.44 76.454) (layer Edge.Cuts) (width 0.05))
 (segment (start 117.312 107.914) (end 117.602 108.204) (width 1) (layer B.Cu) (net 11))
 (segment (start 117.312 100.838) (end 117.312 107.914) (width 1) (layer B.Cu) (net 11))
 (segment (start 113.03 108.204) (end 117.602 108.204) (width 1) (layer B.Cu) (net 11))
 (segment (start 108.79 94.058) (end 108.712 93.98) (width 1) (layer B.Cu) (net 4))
 (segment (start 112.588 94.058) (end 108.79 94.058) (width 1) (layer B.Cu) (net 4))
 (segment (start 123.531998 110.744) (end 123.952 110.744) (width 1) (layer B.Cu) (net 4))
 (segment (start 105.918 110.744) (end 123.531998 110.744) (width 1) (layer B.Cu) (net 4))
 (segment (start 122.174 80.772) (end 122.174 81.788) (width 1) (layer B.Cu) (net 4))
 (segment (start 122.174 81.788) (end 119.888 84.074) (width 1) (layer B.Cu) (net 4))
 (segment (start 119.888 84.074) (end 119.126 84.074) (width 1) (layer B.Cu) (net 4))
 (segment (start 116.078 87.122) (end 116.078 92.71) (width 1) (layer B.Cu) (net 4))
 (segment (start 114.73 94.058) (end 112.588 94.058) (width 1) (layer B.Cu) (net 4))
 (segment (start 116.078 92.71) (end 114.73 94.058) (width 1) (layer B.Cu) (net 4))
 (segment (start 100.584 85.344) (end 104.648 85.344) (width 1) (layer B.Cu) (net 4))
 (segment (start 114.173 84.455) (end 116.459 86.741) (width 1) (layer B.Cu) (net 4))
 (segment (start 105.537 84.455) (end 114.173 84.455) (width 1) (layer B.Cu) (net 4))
 (segment (start 104.648 85.344) (end 105.537 84.455) (width 1) (layer B.Cu) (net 4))
 (segment (start 119.126 84.074) (end 116.459 86.741) (width 1) (layer B.Cu) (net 4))
 (segment (start 116.459 86.741) (end 116.078 87.122) (width 1) (layer B.Cu) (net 4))
 (segment (start 104.394 83.312) (end 105.537 84.455) (width 1) (layer B.Cu) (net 4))
 (segment (start 104.394 80.518) (end 104.394 83.312) (width 1) (layer B.Cu) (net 4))
 (segment (start 105.918 110.744) (end 104.14 110.744) (width 1) (layer B.Cu) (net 4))
 (segment (start 104.14 110.744) (end 97.79 104.394) (width 1) (layer B.Cu) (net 4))
 (segment (start 97.79 88.138) (end 100.584 85.344) (width 1) (layer B.Cu) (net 4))
 (segment (start 97.79 104.394) (end 97.79 88.138) (width 1) (layer B.Cu) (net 4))
 (segment (start 117.094 80.772) (end 117.094 82.296) (width 1) (layer B.Cu) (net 2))
 (segment (start 117.094 82.296) (end 116.586 82.804) (width 1) (layer B.Cu) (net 2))
 (segment (start 109.22 82.804) (end 106.934 80.518) (width 1) (layer B.Cu) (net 2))
 (segment (start 116.586 82.804) (end 109.22 82.804) (width 1) (layer B.Cu) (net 2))
 (segment (start 120.286 86.36) (end 120.208 86.438) (width 1) (layer B.Cu) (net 3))
 (segment (start 124.206 86.36) (end 120.286 86.36) (width 1) (layer B.Cu) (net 3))
 (segment (start 119.312 98.484) (end 119.312 100.838) (width 1) (layer B.Cu) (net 3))
 (segment (start 117.856 97.028) (end 119.312 98.484) (width 1) (layer B.Cu) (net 3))
 (segment (start 117.856 87.63) (end 117.856 97.028) (width 1) (layer B.Cu) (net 3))
 (segment (start 120.208 86.438) (end 119.048 86.438) (width 1) (layer B.Cu) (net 3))
 (segment (start 119.048 86.438) (end 117.856 87.63) (width 1) (layer B.Cu) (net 3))
 (segment (start 117.856 97.028) (end 111.506 97.028) (width 1) (layer B.Cu) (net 3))
 (segment (start 111.506 97.028) (end 109.728 98.806) (width 1) (layer B.Cu) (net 3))
 (segment (start 109.728 98.806) (end 109.728 106.934) (width 1) (layer B.Cu) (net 3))
 (segment (start 108.458 108.204) (end 105.918 108.204) (width 1) (layer B.Cu) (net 3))
 (segment (start 109.728 106.934) (end 108.458 108.204) (width 1) (layer B.Cu) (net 3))
 (segment (start 105.918 108.204) (end 103.886 108.204) (width 1) (layer B.Cu) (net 3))
 (segment (start 100.48 104.798) (end 100.48 102.798) (width 1) (layer B.Cu) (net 3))
 (segment (start 103.886 108.204) (end 100.48 104.798) (width 1) (layer B.Cu) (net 3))
 (segment (start 125.476 85.09) (end 124.206 86.36) (width 1) (layer B.Cu) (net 3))
 (segment (start 119.634 79.502) (end 120.65 78.486) (width 1) (layer B.Cu) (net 3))
 (segment (start 119.634 80.772) (end 119.634 79.502) (width 1) (layer B.Cu) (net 3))
 (segment (start 120.65 78.486) (end 124.714 78.486) (width 1) (layer B.Cu) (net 3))
 (segment (start 124.714 78.486) (end 125.476 79.248) (width 1) (layer B.Cu) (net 3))
 (segment (start 125.476 79.248) (end 125.476 85.09) (width 1) (layer B.Cu) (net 3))
 (segment (start 114.554 80.772) (end 114.554 78.74) (width 0.5) (layer B.Cu) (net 1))
 (segment (start 114.554 78.74) (end 116.078 77.216) (width 0.5) (layer B.Cu) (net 1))
 (segment (start 126.492 110.744) (end 126.492 97.282) (width 0.5) (layer B.Cu) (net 1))
 (segment (start 126.492 97.282) (end 127.762 96.012) (width 0.5) (layer B.Cu) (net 1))
 (segment (start 127.762 78.74) (end 126.238 77.216) (width 0.5) (layer B.Cu) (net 1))
 (segment (start 127.762 96.012) (end 127.762 78.74) (width 0.5) (layer B.Cu) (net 1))
 (segment (start 116.078 77.216) (end 126.238 77.216) (width 0.5) (layer B.Cu) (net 1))
 (segment (start 108.79 88.978) (end 108.712 88.9) (width 1) (layer B.Cu) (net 8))
 (segment (start 112.588 88.978) (end 108.79 88.978) (width 1) (layer B.Cu) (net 8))
 (segment (start 107.188 88.9) (end 108.712 88.9) (width 1) (layer B.Cu) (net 8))
 (segment (start 100.584 95.504) (end 107.188 88.9) (width 1) (layer B.Cu) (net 8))
 (segment (start 100.584 98.194) (end 100.48 98.298) (width 1) (layer B.Cu) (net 8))
 (segment (start 100.584 95.504) (end 100.584 98.194) (width 1) (layer B.Cu) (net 8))
 (segment (start 108.79 91.518) (end 108.712 91.44) (width 1) (layer B.Cu) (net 6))
 (segment (start 112.588 91.518) (end 108.79 91.518) (width 1) (layer B.Cu) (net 6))
 (segment (start 105.918 105.664) (end 105.918 92.964) (width 1) (layer B.Cu) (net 6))
 (segment (start 107.442 91.44) (end 108.712 91.44) (width 1) (layer B.Cu) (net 6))
 (segment (start 105.918 92.964) (end 107.442 91.44) (width 1) (layer B.Cu) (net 6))
 (segment (start 120.286 88.9) (end 120.208 88.978) (width 1) (layer B.Cu) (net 5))
 (segment (start 124.206 88.9) (end 120.286 88.9) (width 1) (layer B.Cu) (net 5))
 (segment (start 108.79 86.438) (end 108.712 86.36) (width 1) (layer B.Cu) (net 10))
 (segment (start 112.588 86.438) (end 108.79 86.438) (width 1) (layer B.Cu) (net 10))
 (segment (start 120.286 91.44) (end 120.208 91.518) (width 1) (layer B.Cu) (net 7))
 (segment (start 124.206 91.44) (end 120.286 91.44) (width 1) (layer B.Cu) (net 7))
 (segment (start 120.286 93.98) (end 120.208 94.058) (width 1) (layer B.Cu) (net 9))
 (segment (start 124.206 93.98) (end 120.286 93.98) (width 1) (layer B.Cu) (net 9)))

